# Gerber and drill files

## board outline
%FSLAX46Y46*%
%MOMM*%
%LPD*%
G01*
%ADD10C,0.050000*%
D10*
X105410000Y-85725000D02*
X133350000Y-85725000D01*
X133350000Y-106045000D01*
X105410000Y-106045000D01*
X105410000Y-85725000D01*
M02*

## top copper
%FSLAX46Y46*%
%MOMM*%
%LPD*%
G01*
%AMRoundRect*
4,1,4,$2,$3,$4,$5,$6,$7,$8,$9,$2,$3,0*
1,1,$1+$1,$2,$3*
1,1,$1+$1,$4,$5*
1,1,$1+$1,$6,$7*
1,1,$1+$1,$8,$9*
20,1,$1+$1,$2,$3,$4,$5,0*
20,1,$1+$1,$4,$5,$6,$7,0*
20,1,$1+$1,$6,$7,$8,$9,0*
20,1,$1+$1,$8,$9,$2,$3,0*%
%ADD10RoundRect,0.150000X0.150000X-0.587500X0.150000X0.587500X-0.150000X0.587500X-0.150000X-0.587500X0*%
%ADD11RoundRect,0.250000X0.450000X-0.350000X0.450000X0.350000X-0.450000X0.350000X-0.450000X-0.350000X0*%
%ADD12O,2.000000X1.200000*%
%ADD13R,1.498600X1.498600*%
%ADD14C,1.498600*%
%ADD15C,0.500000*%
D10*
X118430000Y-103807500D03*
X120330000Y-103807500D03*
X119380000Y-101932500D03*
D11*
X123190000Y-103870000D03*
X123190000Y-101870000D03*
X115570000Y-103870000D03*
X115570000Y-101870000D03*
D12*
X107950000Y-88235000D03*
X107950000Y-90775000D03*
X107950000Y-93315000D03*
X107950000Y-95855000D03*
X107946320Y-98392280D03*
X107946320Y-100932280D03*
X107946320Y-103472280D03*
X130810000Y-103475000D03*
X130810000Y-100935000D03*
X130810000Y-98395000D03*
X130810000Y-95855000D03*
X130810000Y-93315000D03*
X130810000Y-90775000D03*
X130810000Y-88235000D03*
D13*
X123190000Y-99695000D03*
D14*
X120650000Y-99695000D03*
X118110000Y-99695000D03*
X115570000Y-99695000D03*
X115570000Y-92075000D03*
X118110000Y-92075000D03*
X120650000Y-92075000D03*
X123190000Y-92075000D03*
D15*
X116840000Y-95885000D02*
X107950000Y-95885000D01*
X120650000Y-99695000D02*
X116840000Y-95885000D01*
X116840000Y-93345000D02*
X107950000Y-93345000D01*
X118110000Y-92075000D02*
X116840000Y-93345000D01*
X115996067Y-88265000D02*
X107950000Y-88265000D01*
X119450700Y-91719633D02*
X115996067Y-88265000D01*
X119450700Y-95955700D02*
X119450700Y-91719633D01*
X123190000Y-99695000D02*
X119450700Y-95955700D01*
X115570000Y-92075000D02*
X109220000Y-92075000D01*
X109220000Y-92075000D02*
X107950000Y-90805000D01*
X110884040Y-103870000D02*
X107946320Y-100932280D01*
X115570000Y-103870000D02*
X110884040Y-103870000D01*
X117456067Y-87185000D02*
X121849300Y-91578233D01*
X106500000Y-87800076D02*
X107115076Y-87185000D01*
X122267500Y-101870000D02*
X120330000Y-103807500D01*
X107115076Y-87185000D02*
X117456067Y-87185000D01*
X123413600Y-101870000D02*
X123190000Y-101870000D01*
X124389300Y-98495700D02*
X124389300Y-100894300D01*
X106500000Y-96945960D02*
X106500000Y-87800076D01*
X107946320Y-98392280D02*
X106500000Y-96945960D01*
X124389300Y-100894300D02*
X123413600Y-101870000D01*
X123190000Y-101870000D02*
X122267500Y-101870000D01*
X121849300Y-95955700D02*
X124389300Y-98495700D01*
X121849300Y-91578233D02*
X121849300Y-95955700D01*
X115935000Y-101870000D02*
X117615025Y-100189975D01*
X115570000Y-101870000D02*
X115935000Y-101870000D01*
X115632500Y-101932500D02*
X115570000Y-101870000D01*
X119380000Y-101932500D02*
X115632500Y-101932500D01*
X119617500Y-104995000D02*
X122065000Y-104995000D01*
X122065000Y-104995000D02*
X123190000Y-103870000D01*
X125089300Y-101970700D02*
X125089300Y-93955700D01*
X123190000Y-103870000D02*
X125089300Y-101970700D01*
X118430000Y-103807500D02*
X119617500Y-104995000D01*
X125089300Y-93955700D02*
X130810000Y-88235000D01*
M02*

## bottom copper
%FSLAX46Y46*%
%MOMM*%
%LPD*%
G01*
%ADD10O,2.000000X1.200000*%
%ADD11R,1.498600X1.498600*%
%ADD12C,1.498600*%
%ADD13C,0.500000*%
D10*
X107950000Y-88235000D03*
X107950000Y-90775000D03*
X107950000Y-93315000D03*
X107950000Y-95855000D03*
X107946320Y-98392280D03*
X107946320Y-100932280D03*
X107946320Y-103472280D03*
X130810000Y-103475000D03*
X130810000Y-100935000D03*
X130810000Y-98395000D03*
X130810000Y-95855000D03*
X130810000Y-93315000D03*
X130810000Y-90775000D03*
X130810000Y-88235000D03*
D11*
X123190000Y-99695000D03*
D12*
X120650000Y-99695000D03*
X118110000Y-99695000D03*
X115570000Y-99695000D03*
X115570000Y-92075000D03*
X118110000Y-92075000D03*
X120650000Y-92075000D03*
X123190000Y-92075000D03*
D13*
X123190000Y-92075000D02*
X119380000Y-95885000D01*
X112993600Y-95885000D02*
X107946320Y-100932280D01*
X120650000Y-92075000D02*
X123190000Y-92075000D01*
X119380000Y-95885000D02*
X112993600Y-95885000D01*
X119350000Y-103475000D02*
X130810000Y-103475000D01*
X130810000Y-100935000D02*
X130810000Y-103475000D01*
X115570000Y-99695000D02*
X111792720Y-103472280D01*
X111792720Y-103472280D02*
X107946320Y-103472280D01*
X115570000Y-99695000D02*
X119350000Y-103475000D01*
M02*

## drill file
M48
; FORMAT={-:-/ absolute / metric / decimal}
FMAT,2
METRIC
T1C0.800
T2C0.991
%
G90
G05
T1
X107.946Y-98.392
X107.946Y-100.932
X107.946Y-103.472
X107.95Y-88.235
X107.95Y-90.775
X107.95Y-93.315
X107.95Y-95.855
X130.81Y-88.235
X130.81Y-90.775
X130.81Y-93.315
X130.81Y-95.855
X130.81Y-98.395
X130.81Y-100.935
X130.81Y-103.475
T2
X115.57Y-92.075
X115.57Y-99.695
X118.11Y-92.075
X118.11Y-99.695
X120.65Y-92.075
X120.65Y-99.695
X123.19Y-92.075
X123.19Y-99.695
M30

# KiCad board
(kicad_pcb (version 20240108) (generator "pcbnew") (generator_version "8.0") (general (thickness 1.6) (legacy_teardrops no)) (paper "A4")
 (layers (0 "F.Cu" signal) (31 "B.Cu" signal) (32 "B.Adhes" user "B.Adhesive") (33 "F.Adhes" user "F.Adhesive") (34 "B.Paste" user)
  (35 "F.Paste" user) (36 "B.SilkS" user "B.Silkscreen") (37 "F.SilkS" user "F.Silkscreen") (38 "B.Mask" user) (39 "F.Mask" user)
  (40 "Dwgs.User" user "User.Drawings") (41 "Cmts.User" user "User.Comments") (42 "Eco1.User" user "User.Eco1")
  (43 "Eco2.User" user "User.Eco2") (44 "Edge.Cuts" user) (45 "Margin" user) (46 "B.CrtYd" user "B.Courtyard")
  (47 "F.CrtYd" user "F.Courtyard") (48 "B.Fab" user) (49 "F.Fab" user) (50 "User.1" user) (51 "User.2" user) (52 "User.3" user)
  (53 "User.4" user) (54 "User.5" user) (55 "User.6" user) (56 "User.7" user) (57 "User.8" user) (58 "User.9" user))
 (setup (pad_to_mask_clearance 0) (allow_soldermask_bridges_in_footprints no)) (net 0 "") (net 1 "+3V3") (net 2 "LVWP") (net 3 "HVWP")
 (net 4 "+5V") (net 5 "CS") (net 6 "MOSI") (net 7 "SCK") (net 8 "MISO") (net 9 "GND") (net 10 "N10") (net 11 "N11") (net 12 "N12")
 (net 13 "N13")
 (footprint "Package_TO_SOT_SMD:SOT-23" (layer "F.Cu") (at 119.38 102.87 90)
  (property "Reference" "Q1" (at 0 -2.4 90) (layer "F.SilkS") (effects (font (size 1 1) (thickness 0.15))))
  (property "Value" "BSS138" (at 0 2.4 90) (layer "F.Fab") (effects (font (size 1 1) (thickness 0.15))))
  (pad "1" smd roundrect (at -0.9375 -0.95 90) (size 1.475 0.6) (layers "F.Cu" "F.Paste" "F.Mask") (roundrect_rratio 0.25) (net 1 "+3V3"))
  (pad "2" smd roundrect (at -0.9375 0.95 90) (size 1.475 0.6) (layers "F.Cu" "F.Paste" "F.Mask") (roundrect_rratio 0.25) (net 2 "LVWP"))
  (pad "3" smd roundrect (at 0.9375 0 90) (size 1.475 0.6) (layers "F.Cu" "F.Paste" "F.Mask") (roundrect_rratio 0.25) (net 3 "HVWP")))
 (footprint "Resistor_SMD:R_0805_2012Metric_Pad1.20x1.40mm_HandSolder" (layer "F.Cu") (at 123.19 102.87 90)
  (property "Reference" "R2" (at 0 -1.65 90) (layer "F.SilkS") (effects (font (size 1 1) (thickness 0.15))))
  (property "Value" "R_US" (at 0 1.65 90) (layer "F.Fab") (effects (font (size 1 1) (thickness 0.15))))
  (pad "1" smd roundrect (at -1 0 90) (size 1.2 1.4) (layers "F.Cu" "F.Paste" "F.Mask") (roundrect_rratio 0.208333) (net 1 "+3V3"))
  (pad "2" smd roundrect (at 1 0 90) (size 1.2 1.4) (layers "F.Cu" "F.Paste" "F.Mask") (roundrect_rratio 0.208333) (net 2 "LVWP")))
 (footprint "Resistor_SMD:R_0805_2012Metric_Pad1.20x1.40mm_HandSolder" (layer "F.Cu") (at 115.57 102.87 90)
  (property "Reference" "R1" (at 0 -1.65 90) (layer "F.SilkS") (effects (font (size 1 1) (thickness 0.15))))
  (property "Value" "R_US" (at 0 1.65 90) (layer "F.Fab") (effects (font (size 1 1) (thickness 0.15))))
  (pad "1" smd roundrect (at -1 0 90) (size 1.2 1.4) (layers "F.Cu" "F.Paste" "F.Mask") (roundrect_rratio 0.208333) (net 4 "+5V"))
  (pad "2" smd roundrect (at 1 0 90) (size 1.2 1.4) (layers "F.Cu" "F.Paste" "F.Mask") (roundrect_rratio 0.208333) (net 3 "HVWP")))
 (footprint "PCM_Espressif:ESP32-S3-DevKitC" (layer "F.Cu") (at 107.95 88.135)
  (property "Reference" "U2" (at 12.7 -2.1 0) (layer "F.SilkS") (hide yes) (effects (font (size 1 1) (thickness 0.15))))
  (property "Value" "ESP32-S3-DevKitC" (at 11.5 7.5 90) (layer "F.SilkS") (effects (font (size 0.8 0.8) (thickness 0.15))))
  (pad "16" thru_hole oval (at 0 0.1 270) (size 1.2 2) (drill 0.8) (layers "*.Cu" "*.Mask") (remove_unused_layers no) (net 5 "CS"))
  (pad "17" thru_hole oval (at 0 2.64 270) (size 1.2 2) (drill 0.8) (layers "*.Cu" "*.Mask") (remove_unused_layers no) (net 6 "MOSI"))
  (pad "18" thru_hole oval (at 0 5.18 270) (size 1.2 2) (drill 0.8) (layers "*.Cu" "*.Mask") (remove_unused_layers no) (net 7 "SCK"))
  (pad "19" thru_hole oval (at 0 7.72 270) (size 1.2 2) (drill 0.8) (layers "*.Cu" "*.Mask") (remove_unused_layers no) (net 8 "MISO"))
  (pad "20" thru_hole oval (at -0.00368 10.25728 270) (size 1.2 2) (drill 0.8) (layers "*.Cu" "*.Mask") (remove_unused_layers no)
   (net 2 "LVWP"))
  (pad "21" thru_hole oval (at -0.00368 12.79728 270) (size 1.2 2) (drill 0.8) (layers "*.Cu" "*.Mask") (remove_unused_layers no)
   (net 4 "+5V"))
  (pad "22" thru_hole oval (at -0.00368 15.33728 270) (size 1.2 2) (drill 0.8) (layers "*.Cu" "*.Mask") (remove_unused_layers no)
   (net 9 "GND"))
  (pad "23" thru_hole oval (at 22.86 15.34 270) (size 1.2 2) (drill 0.8) (layers "*.Cu" "*.Mask") (remove_unused_layers no) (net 9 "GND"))
  (pad "24" thru_hole oval (at 22.86 12.8 270) (size 1.2 2) (drill 0.8) (layers "*.Cu" "*.Mask") (remove_unused_layers no) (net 9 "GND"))
  (pad "25" thru_hole oval (at 22.86 10.26 270) (size 1.2 2) (drill 0.8) (layers "*.Cu" "*.Mask") (remove_unused_layers no) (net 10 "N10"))
  (pad "26" thru_hole oval (at 22.86 7.72 270) (size 1.2 2) (drill 0.8) (layers "*.Cu" "*.Mask") (remove_unused_layers no) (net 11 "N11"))
  (pad "27" thru_hole oval (at 22.86 5.18 270) (size 1.2 2) (drill 0.8) (layers "*.Cu" "*.Mask") (remove_unused_layers no) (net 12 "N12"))
  (pad "28" thru_hole oval (at 22.86 2.64 270) (size 1.2 2) (drill 0.8) (layers "*.Cu" "*.Mask") (remove_unused_layers no) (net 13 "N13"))
  (pad "29" thru_hole oval (at 22.86 0.1 270) (size 1.2 2) (drill 0.8) (layers "*.Cu" "*.Mask") (remove_unused_layers no) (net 1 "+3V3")))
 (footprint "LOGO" (layer "B.Cu") (at 111.76 88.9 90)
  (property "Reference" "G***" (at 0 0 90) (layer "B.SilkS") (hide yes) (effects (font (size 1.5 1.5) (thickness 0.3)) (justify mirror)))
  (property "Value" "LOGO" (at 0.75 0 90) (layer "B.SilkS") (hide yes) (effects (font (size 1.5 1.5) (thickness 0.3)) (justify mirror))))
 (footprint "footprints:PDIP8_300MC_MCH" (layer "B.Cu") (at 123.19 99.695 90)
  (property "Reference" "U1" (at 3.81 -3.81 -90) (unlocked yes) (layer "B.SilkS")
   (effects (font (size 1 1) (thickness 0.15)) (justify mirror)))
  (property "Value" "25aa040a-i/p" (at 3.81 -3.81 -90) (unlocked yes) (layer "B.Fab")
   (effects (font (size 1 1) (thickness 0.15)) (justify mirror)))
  (pad "1" thru_hole rect (at 0 0 90) (size 1.4986 1.4986) (drill 0.9906) (layers "*.Cu" "*.Mask") (remove_unused_layers no) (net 5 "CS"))
  (pad "2" thru_hole circle (at 0 -2.54 90) (size 1.4986 1.4986) (drill 0.9906) (layers "*.Cu" "*.Mask") (remove_unused_layers no)
   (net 8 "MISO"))
  (pad "3" thru_hole circle (at 0 -5.08 90) (size 1.4986 1.4986) (drill 0.9906) (layers "*.Cu" "*.Mask") (remove_unused_layers no)
   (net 3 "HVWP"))
  (pad "4" thru_hole circle (at 0 -7.62 90) (size 1.4986 1.4986) (drill 0.9906) (layers "*.Cu" "*.Mask") (remove_unused_layers no)
   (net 9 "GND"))
  (pad "5" thru_hole circle (at 7.62 -7.62 90) (size 1.4986 1.4986) (drill 0.9906) (layers "*.Cu" "*.Mask") (remove_unused_layers no)
   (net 6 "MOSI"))
  (pad "6" thru_hole circle (at 7.62 -5.08 90) (size 1.4986 1.4986) (drill 0.9906) (layers "*.Cu" "*.Mask") (remove_unused_layers no)
   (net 7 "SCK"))
  (pad "7" thru_hole circle (at 7.62 -2.54 90) (size 1.4986 1.4986) (drill 0.9906) (layers "*.Cu" "*.Mask") (remove_unused_layers no)
   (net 4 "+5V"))
  (pad "8" thru_hole circle (at 7.62 0 90) (size 1.4986 1.4986) (drill 0.9906) (layers "*.Cu" "*.Mask") (remove_unused_layers no)
   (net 4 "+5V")))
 (gr_rect (start 105.41 85.725) (end 133.35 106.045) (stroke (width 0.05) (type default)) (fill none) (layer "Edge.Cuts"))
 (segment (start 116.84 95.885) (end 107.95 95.885) (width 0.5) (layer "F.Cu") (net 8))
 (segment (start 120.65 99.695) (end 116.84 95.885) (width 0.5) (layer "F.Cu") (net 8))
 (segment (start 116.84 93.345) (end 107.95 93.345) (width 0.5) (layer "F.Cu") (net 7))
 (segment (start 118.11 92.075) (end 116.84 93.345) (width 0.5) (layer "F.Cu") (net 7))
 (segment (start 115.996067 88.265) (end 107.95 88.265) (width 0.5) (layer "F.Cu") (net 5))
 (segment (start 119.4507 91.719633) (end 115.996067 88.265) (width 0.5) (layer "F.Cu") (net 5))
 (segment (start 119.4507 95.9557) (end 119.4507 91.719633) (width 0.5) (layer "F.Cu") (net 5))
 (segment (start 123.19 99.695) (end 119.4507 95.9557) (width 0.5) (layer "F.Cu") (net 5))
 (segment (start 115.57 92.075) (end 109.22 92.075) (width 0.5) (layer "F.Cu") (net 6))
 (segment (start 109.22 92.075) (end 107.95 90.805) (width 0.5) (layer "F.Cu") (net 6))
 (segment (start 110.88404 103.87) (end 107.94632 100.93228) (width 0.5) (layer "F.Cu") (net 4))
 (segment (start 115.57 103.87) (end 110.88404 103.87) (width 0.5) (layer "F.Cu") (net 4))
 (segment (start 123.19 92.075) (end 119.38 95.885) (width 0.5) (layer "B.Cu") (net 4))
 (segment (start 112.9936 95.885) (end 107.94632 100.93228) (width 0.5) (layer "B.Cu") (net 4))
 (segment (start 120.65 92.075) (end 123.19 92.075) (width 0.5) (layer "B.Cu") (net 4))
 (segment (start 119.38 95.885) (end 112.9936 95.885) (width 0.5) (layer "B.Cu") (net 4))
 (segment (start 119.35 103.475) (end 130.81 103.475) (width 0.5) (layer "B.Cu") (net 9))
 (segment (start 130.81 100.935) (end 130.81 103.475) (width 0.5) (layer "B.Cu") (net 9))
 (segment (start 115.57 99.695) (end 111.79272 103.47228) (width 0.5) (layer "B.Cu") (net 9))
 (segment (start 111.79272 103.47228) (end 107.94632 103.47228) (width 0.5) (layer "B.Cu") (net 9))
 (segment (start 115.57 99.695) (end 119.35 103.475) (width 0.5) (layer "B.Cu") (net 9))
 (segment (start 117.456067 87.185) (end 121.8493 91.578233) (width 0.5) (layer "F.Cu") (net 2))
 (segment (start 106.5 87.800076) (end 107.115076 87.185) (width 0.5) (layer "F.Cu") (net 2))
 (segment (start 122.2675 101.87) (end 120.33 103.8075) (width 0.5) (layer "F.Cu") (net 2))
 (segment (start 107.115076 87.185) (end 117.456067 87.185) (width 0.5) (layer "F.Cu") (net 2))
 (segment (start 123.4136 101.87) (end 123.19 101.87) (width 0.5) (layer "F.Cu") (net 2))
 (segment (start 124.3893 98.4957) (end 124.3893 100.8943) (width 0.5) (layer "F.Cu") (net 2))
 (segment (start 106.5 96.94596) (end 106.5 87.800076) (width 0.5) (layer "F.Cu") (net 2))
 (segment (start 107.94632 98.39228) (end 106.5 96.94596) (width 0.5) (layer "F.Cu") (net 2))
 (segment (start 124.3893 100.8943) (end 123.4136 101.87) (width 0.5) (layer "F.Cu") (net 2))
 (segment (start 123.19 101.87) (end 122.2675 101.87) (width 0.5) (layer "F.Cu") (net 2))
 (segment (start 121.8493 95.9557) (end 124.3893 98.4957) (width 0.5) (layer "F.Cu") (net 2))
 (segment (start 121.8493 91.578233) (end 121.8493 95.9557) (width 0.5) (layer "F.Cu") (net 2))
 (segment (start 115.935 101.87) (end 117.615025 100.189975) (width 0.5) (layer "F.Cu") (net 3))
 (segment (start 115.57 101.87) (end 115.935 101.87) (width 0.5) (layer "F.Cu") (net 3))
 (segment (start 115.6325 101.9325) (end 115.57 101.87) (width 0.5) (layer "F.Cu") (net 3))
 (segment (start 119.38 101.9325) (end 115.6325 101.9325) (width 0.5) (layer "F.Cu") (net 3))
 (segment (start 119.6175 104.995) (end 122.065 104.995) (width 0.5) (layer "F.Cu") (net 1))
 (segment (start 122.065 104.995) (end 123.19 103.87) (width 0.5) (layer "F.Cu") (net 1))
 (segment (start 125.0893 101.9707) (end 125.0893 93.9557) (width 0.5) (layer "F.Cu") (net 1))
 (segment (start 123.19 103.87) (end 125.0893 101.9707) (width 0.5) (layer "F.Cu") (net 1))
 (segment (start 118.43 103.8075) (end 119.6175 104.995) (width 0.5) (layer "F.Cu") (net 1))
 (segment (start 125.0893 93.9557) (end 130.81 88.235) (width 0.5) (layer "F.Cu") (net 1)))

